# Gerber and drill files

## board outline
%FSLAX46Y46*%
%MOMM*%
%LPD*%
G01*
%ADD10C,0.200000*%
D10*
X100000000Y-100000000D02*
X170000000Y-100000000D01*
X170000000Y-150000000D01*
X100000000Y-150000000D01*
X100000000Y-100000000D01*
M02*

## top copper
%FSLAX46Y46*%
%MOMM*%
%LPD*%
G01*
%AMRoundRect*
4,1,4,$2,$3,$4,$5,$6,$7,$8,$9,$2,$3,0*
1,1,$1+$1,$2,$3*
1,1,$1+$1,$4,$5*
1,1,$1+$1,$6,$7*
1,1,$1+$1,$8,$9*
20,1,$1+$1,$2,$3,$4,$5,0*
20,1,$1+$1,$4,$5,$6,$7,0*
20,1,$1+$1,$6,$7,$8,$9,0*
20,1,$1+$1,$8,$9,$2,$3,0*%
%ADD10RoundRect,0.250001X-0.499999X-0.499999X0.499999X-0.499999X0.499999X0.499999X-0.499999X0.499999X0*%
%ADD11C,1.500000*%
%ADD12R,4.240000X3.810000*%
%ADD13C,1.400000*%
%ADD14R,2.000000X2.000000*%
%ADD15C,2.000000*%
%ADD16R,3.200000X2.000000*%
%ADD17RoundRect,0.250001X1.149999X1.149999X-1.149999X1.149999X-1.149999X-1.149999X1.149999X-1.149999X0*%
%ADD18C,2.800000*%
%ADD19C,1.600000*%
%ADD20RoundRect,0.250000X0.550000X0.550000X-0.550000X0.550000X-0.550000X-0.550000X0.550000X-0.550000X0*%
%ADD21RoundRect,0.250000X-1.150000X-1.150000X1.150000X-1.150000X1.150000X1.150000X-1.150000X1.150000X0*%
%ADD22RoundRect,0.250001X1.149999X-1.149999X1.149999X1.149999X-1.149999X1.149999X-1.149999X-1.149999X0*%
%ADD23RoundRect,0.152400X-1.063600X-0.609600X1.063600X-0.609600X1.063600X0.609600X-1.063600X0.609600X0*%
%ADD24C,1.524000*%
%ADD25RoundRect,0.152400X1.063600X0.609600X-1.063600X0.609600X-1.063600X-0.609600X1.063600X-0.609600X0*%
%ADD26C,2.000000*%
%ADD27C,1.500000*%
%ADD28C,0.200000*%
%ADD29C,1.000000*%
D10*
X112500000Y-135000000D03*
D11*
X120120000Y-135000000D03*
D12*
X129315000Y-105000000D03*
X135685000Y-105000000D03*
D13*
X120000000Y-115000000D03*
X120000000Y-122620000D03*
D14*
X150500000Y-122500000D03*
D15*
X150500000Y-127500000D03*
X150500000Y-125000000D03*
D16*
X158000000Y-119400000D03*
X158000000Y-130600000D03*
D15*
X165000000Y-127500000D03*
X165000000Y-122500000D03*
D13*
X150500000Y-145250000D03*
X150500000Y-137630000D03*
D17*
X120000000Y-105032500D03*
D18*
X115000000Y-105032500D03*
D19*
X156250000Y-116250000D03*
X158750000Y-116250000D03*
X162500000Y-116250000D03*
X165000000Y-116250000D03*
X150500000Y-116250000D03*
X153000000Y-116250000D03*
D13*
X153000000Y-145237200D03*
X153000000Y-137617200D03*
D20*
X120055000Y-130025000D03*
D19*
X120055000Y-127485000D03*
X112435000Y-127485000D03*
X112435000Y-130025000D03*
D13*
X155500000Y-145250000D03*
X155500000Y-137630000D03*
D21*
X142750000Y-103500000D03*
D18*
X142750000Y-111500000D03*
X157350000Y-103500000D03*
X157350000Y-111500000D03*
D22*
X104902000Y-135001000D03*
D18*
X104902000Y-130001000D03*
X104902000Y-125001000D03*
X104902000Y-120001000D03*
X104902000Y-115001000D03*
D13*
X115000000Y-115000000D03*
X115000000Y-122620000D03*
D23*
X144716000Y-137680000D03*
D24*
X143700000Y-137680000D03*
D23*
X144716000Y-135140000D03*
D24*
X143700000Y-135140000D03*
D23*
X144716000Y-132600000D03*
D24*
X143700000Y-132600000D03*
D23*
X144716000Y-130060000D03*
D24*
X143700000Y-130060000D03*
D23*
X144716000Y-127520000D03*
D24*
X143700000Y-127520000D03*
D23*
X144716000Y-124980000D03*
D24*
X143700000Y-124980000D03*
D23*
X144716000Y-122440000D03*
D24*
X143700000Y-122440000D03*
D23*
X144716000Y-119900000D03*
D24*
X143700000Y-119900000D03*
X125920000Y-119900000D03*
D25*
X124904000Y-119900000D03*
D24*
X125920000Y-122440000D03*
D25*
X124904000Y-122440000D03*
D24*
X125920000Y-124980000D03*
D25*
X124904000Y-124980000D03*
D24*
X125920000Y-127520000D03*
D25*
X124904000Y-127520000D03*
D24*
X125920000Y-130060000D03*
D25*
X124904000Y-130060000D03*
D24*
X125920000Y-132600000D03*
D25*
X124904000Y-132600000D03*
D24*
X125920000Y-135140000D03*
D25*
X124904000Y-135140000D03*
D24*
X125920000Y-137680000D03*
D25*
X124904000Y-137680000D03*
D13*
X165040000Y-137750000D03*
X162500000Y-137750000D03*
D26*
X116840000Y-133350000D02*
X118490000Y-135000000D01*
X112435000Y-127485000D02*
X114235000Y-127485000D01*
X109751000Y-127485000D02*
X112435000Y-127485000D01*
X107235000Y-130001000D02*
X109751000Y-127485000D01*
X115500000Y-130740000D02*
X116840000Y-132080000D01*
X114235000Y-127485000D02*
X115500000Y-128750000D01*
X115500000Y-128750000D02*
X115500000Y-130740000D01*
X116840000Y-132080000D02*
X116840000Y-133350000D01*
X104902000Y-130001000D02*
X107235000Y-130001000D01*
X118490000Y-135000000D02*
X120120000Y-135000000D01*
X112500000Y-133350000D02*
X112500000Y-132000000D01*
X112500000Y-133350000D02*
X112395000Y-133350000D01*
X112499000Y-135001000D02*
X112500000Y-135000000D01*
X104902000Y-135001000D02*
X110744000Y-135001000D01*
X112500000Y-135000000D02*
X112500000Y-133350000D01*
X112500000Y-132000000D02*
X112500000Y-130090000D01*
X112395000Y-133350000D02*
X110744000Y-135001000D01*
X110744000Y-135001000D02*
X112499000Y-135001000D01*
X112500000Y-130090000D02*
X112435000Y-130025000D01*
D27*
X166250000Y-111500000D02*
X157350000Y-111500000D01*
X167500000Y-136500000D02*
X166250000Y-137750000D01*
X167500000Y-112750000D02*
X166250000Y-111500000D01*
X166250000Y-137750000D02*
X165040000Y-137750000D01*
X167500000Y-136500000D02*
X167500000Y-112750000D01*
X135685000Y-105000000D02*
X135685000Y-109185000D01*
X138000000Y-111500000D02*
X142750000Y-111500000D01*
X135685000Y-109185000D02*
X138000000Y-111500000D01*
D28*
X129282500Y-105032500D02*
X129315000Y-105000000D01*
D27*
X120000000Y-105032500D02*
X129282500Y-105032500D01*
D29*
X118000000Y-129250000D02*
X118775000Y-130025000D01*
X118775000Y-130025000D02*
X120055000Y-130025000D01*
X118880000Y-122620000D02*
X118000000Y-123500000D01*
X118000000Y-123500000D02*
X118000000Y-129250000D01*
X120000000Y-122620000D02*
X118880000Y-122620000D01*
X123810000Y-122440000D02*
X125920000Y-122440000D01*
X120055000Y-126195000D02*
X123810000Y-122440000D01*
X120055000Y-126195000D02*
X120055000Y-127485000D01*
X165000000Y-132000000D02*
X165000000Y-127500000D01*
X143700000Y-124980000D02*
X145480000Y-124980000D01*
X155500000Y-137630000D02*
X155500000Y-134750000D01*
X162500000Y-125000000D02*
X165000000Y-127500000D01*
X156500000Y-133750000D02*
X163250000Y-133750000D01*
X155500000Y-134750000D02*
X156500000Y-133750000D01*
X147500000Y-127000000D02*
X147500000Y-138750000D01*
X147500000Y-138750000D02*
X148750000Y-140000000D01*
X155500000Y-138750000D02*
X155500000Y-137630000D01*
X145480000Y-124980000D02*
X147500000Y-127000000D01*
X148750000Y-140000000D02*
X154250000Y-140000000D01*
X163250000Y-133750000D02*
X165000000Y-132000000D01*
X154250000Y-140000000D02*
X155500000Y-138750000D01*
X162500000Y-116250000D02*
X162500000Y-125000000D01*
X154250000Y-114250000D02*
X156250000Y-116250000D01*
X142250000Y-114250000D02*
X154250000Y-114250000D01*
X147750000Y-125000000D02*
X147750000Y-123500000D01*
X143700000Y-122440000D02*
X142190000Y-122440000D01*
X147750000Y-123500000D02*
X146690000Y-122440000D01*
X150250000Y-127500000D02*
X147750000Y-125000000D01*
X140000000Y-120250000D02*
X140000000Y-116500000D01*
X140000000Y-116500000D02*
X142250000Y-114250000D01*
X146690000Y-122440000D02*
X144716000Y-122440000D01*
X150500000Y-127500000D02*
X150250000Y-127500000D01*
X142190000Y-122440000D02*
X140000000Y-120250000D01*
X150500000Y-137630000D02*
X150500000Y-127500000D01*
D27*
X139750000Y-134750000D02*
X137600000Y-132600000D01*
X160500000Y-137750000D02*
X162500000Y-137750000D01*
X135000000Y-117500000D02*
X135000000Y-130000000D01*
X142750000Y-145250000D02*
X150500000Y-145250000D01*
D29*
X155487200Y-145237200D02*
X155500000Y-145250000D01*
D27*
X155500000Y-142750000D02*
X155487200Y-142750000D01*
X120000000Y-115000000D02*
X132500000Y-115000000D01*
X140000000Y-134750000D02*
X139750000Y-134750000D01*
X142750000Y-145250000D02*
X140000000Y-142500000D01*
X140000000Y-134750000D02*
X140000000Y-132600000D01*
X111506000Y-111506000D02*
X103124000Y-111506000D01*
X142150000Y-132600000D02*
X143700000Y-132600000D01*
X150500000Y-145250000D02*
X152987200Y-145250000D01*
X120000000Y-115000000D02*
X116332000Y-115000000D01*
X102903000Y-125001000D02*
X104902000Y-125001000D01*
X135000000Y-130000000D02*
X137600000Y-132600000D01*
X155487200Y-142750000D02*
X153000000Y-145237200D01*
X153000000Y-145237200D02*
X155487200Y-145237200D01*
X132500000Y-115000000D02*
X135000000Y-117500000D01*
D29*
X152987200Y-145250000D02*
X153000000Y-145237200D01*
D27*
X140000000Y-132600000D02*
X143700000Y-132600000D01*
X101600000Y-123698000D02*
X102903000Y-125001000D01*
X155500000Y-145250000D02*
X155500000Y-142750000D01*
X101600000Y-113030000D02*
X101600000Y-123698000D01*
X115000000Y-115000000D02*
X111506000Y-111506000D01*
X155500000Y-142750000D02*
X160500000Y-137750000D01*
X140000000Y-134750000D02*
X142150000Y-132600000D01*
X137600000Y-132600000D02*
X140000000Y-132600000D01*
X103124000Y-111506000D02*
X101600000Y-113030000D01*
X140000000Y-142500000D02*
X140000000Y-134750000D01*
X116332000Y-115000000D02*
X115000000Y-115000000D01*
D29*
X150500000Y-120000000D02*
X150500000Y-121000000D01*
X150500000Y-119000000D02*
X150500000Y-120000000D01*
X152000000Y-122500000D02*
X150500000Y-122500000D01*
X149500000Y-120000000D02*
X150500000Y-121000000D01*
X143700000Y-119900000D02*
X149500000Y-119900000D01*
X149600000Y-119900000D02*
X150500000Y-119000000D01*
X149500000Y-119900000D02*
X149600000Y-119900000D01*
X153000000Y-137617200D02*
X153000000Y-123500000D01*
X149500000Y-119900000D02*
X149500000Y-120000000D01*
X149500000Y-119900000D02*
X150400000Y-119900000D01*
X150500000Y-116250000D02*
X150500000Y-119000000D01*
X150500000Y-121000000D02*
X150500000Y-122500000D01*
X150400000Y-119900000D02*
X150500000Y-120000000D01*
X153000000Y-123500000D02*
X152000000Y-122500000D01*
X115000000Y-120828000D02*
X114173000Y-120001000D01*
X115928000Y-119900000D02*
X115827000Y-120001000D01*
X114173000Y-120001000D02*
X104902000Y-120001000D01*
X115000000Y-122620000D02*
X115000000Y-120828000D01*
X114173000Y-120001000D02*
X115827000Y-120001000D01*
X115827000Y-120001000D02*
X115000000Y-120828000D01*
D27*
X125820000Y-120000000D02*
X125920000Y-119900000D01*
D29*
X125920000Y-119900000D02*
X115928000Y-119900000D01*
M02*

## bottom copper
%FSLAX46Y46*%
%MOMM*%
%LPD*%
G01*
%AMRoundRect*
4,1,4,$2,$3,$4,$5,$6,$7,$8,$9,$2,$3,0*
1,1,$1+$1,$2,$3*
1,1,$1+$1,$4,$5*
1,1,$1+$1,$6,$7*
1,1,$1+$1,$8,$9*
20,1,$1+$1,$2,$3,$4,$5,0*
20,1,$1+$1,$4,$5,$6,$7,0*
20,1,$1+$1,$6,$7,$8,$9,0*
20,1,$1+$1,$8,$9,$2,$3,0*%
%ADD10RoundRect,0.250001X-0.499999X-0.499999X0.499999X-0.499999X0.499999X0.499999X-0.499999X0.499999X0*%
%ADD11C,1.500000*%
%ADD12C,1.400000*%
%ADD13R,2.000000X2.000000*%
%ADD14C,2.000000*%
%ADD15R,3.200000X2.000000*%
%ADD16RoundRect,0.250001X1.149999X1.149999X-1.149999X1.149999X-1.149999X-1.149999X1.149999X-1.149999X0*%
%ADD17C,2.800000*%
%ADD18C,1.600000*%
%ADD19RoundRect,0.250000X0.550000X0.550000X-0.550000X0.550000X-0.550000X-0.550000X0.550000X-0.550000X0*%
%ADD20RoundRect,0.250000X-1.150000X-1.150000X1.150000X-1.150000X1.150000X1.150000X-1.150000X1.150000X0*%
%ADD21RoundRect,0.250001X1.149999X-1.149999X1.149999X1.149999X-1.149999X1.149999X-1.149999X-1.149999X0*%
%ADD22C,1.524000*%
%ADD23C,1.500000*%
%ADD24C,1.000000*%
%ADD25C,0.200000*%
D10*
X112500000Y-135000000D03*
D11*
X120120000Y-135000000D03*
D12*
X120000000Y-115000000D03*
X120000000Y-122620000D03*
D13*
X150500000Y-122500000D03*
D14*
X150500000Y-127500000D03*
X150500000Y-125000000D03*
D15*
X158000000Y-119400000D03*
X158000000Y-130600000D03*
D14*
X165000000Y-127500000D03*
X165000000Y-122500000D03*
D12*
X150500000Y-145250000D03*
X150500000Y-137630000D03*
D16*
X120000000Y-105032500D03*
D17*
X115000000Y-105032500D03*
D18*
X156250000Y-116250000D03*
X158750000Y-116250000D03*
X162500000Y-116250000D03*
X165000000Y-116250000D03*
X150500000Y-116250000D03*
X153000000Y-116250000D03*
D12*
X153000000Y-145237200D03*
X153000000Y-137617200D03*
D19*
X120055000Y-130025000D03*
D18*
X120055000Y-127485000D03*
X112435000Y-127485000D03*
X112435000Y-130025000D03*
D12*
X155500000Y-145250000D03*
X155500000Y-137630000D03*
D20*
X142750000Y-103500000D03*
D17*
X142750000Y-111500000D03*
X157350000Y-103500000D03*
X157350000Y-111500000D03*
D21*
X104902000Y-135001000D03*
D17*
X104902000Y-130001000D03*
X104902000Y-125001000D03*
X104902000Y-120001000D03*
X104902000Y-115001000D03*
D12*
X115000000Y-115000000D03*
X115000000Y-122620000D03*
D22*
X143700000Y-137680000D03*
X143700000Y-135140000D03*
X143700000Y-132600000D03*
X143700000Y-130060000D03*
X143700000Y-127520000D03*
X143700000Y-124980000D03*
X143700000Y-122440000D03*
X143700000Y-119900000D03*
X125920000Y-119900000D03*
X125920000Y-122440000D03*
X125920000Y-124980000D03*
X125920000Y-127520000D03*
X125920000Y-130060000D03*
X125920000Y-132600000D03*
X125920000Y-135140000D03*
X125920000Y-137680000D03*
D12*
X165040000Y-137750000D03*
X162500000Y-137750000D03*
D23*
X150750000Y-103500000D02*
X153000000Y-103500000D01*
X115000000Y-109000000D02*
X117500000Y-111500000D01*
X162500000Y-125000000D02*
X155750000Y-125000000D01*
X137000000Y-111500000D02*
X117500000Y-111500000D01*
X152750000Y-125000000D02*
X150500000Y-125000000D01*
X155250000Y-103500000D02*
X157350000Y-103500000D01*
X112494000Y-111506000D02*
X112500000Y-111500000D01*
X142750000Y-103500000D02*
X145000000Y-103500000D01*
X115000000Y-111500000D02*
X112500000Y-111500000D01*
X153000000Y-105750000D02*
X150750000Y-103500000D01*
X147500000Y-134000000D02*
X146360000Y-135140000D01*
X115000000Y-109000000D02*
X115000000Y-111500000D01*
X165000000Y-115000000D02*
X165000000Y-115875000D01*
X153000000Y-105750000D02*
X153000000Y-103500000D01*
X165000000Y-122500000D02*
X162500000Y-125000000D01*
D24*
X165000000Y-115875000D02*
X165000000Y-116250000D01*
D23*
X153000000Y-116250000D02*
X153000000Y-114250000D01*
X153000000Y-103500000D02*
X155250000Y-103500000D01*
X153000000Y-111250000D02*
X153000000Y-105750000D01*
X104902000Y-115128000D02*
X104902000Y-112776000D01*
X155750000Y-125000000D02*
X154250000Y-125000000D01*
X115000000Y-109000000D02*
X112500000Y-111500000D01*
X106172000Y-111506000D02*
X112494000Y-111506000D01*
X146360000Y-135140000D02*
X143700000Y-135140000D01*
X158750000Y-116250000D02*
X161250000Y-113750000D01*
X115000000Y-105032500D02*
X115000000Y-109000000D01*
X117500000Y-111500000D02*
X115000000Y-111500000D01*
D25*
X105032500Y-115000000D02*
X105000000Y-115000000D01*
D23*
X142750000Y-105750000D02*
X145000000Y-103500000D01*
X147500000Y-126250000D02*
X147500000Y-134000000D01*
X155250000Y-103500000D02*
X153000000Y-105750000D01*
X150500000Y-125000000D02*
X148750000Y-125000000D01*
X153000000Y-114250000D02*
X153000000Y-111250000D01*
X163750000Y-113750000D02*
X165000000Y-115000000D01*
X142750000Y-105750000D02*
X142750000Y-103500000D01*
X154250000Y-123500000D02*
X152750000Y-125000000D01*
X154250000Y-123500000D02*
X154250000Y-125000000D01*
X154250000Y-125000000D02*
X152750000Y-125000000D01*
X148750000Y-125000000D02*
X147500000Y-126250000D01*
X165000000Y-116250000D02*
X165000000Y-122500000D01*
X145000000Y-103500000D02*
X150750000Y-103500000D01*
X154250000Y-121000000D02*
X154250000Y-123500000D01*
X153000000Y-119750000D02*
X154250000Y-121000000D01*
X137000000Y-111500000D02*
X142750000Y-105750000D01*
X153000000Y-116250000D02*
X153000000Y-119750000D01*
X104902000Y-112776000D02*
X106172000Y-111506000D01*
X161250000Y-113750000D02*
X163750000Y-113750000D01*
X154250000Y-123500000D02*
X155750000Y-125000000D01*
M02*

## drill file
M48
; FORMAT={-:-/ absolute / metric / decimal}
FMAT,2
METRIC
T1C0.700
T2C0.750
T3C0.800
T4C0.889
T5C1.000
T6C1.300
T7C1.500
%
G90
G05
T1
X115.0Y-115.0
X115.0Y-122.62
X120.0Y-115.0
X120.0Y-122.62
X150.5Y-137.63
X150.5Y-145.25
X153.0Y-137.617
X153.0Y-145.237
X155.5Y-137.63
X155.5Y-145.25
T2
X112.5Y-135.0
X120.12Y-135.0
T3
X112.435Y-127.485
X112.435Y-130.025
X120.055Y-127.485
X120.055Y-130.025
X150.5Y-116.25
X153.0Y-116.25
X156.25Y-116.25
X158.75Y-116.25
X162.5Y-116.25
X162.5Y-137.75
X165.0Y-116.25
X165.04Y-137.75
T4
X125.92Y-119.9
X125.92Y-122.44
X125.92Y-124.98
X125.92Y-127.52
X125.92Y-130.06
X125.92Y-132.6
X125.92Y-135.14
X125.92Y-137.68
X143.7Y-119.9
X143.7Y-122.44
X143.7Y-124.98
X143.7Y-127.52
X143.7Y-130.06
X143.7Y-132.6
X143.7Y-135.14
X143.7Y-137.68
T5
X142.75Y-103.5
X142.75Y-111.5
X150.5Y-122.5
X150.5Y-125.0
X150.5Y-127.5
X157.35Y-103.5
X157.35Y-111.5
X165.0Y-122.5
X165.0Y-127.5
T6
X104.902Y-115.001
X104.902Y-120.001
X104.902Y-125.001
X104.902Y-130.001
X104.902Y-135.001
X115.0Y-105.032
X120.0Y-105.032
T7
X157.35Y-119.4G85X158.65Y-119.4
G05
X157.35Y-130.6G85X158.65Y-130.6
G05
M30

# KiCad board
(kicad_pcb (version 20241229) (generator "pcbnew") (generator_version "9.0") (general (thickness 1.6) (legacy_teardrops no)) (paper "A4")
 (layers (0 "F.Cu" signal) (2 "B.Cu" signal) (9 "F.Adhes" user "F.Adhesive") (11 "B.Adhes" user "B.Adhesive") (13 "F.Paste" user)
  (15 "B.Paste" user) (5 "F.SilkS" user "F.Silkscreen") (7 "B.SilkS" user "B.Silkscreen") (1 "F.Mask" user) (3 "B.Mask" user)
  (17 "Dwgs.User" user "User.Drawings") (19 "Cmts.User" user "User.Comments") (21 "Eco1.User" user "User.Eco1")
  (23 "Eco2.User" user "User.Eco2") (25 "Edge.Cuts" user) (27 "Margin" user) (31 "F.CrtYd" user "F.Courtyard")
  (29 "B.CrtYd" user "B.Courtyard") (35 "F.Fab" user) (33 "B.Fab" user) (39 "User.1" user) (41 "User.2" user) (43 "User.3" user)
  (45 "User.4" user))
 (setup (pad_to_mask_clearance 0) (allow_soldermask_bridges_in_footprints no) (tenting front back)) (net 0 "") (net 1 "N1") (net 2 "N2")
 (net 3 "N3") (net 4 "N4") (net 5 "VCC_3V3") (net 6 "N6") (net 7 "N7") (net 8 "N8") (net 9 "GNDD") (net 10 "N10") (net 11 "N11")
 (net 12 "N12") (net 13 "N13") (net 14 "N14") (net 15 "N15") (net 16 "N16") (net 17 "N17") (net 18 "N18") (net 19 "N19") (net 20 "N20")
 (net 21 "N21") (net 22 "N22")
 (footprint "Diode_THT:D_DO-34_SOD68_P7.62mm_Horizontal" (layer "F.Cu") (at 112.5 135)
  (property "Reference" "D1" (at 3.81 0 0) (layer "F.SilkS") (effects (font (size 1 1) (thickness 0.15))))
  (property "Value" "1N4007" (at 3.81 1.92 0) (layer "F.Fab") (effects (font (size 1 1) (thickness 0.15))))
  (pad "1" thru_hole roundrect (at 0 0) (size 1.5 1.5) (drill 0.75) (layers "*.Cu" "*.Mask") (remove_unused_layers no)
   (roundrect_rratio 0.166667) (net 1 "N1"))
  (pad "2" thru_hole circle (at 7.62 0) (size 1.5 1.5) (drill 0.75) (layers "*.Cu" "*.Mask") (remove_unused_layers no) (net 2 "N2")))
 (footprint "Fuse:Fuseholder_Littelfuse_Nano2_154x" (layer "F.Cu") (at 132.5 105)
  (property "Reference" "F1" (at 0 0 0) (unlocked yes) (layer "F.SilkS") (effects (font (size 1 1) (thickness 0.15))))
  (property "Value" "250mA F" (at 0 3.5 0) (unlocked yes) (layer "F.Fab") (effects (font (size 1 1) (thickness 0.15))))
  (pad "1" smd rect (at -3.185 0) (size 4.24 3.81) (layers "F.Cu" "F.Mask" "F.Paste") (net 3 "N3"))
  (pad "2" smd rect (at 3.185 0) (size 4.24 3.81) (layers "F.Cu" "F.Mask" "F.Paste") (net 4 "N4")))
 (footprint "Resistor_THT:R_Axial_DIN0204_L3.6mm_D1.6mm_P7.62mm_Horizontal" (layer "F.Cu") (at 120 115 -90)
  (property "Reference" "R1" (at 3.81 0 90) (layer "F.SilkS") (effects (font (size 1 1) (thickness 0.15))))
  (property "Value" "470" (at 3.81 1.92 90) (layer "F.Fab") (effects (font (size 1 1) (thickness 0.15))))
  (pad "1" thru_hole circle (at 0 0 270) (size 1.4 1.4) (drill 0.7) (layers "*.Cu" "*.Mask") (remove_unused_layers no) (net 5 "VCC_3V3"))
  (pad "2" thru_hole circle (at 7.62 0 270) (size 1.4 1.4) (drill 0.7) (layers "*.Cu" "*.Mask") (remove_unused_layers no) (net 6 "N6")))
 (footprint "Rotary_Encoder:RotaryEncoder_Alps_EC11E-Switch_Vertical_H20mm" (layer "F.Cu") (at 150.5 122.5)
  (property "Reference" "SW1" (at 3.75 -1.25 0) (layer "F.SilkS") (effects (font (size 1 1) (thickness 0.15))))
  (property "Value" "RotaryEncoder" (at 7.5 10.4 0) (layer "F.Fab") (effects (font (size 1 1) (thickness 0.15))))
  (pad "A" thru_hole rect (at 0 0) (size 2 2) (drill 1) (layers "*.Cu" "*.Mask") (remove_unused_layers no) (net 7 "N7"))
  (pad "B" thru_hole circle (at 0 5) (size 2 2) (drill 1) (layers "*.Cu" "*.Mask") (remove_unused_layers no) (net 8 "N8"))
  (pad "C" thru_hole circle (at 0 2.5) (size 2 2) (drill 1) (layers "*.Cu" "*.Mask") (remove_unused_layers no) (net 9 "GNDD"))
  (pad "MP" thru_hole rect (at 7.5 -3.1) (size 3.2 2) (drill oval 2.8 1.5) (layers "*.Cu" "*.Mask") (remove_unused_layers no))
  (pad "MP" thru_hole rect (at 7.5 8.1) (size 3.2 2) (drill oval 2.8 1.5) (layers "*.Cu" "*.Mask") (remove_unused_layers no))
  (pad "S1" thru_hole circle (at 14.5 5) (size 2 2) (drill 1) (layers "*.Cu" "*.Mask") (remove_unused_layers no) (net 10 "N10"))
  (pad "S2" thru_hole circle (at 14.5 0) (size 2 2) (drill 1) (layers "*.Cu" "*.Mask") (remove_unused_layers no) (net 9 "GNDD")))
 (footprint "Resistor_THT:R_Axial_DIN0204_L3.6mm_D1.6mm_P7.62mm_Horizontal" (layer "F.Cu") (at 150.5 145.25 90)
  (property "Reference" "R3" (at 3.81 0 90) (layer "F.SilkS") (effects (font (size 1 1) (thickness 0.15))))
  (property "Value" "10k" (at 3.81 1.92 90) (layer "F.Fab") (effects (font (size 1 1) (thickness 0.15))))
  (pad "1" thru_hole circle (at 0 0 90) (size 1.4 1.4) (drill 0.7) (layers "*.Cu" "*.Mask") (remove_unused_layers no) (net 5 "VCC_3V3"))
  (pad "2" thru_hole circle (at 7.62 0 90) (size 1.4 1.4) (drill 0.7) (layers "*.Cu" "*.Mask") (remove_unused_layers no) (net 8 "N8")))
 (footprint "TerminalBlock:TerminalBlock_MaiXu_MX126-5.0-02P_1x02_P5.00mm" (layer "F.Cu") (at 120 105.0325 180)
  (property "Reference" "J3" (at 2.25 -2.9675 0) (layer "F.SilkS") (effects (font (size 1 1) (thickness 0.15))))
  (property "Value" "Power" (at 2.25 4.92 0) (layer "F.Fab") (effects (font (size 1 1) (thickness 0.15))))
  (pad "1" thru_hole roundrect (at 0 0 180) (size 2.8 2.8) (drill 1.3) (layers "*.Cu" "*.Mask") (remove_unused_layers no)
   (roundrect_rratio 0.089286) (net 3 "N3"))
  (pad "2" thru_hole circle (at 5 0 180) (size 2.8 2.8) (drill 1.3) (layers "*.Cu" "*.Mask") (remove_unused_layers no) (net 9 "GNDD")))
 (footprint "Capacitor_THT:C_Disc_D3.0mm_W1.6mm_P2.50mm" (layer "F.Cu") (at 156.25 116.25)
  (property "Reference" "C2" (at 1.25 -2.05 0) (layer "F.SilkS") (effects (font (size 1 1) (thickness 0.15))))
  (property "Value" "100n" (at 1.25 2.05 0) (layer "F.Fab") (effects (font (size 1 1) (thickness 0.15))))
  (pad "1" thru_hole circle (at 0 0) (size 1.6 1.6) (drill 0.8) (layers "*.Cu" "*.Mask") (remove_unused_layers no) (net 8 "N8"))
  (pad "2" thru_hole circle (at 2.5 0) (size 1.6 1.6) (drill 0.8) (layers "*.Cu" "*.Mask") (remove_unused_layers no) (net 9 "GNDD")))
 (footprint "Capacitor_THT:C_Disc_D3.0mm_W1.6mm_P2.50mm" (layer "F.Cu") (at 162.5 116.25)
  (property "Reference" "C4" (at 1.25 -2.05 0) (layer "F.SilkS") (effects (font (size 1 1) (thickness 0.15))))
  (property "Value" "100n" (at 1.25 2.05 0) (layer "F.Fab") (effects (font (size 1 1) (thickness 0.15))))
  (pad "1" thru_hole circle (at 0 0) (size 1.6 1.6) (drill 0.8) (layers "*.Cu" "*.Mask") (remove_unused_layers no) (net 10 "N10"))
  (pad "2" thru_hole circle (at 2.5 0) (size 1.6 1.6) (drill 0.8) (layers "*.Cu" "*.Mask") (remove_unused_layers no) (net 9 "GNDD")))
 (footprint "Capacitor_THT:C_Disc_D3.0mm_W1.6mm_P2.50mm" (layer "F.Cu") (at 150.5 116.25)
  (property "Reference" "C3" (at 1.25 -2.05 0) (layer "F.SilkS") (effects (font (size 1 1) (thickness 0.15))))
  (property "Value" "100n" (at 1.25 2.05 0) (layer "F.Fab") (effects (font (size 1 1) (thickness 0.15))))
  (pad "1" thru_hole circle (at 0 0) (size 1.6 1.6) (drill 0.8) (layers "*.Cu" "*.Mask") (remove_unused_layers no) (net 7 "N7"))
  (pad "2" thru_hole circle (at 2.5 0) (size 1.6 1.6) (drill 0.8) (layers "*.Cu" "*.Mask") (remove_unused_layers no) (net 9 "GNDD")))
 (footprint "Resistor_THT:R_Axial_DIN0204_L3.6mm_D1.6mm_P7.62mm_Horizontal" (layer "F.Cu") (at 153 145.2372 90)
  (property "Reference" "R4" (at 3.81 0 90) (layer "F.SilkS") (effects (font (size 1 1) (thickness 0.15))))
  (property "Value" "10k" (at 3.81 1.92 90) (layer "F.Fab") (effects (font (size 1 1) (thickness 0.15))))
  (pad "1" thru_hole circle (at 0 0 90) (size 1.4 1.4) (drill 0.7) (layers "*.Cu" "*.Mask") (remove_unused_layers no) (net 5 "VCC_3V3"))
  (pad "2" thru_hole circle (at 7.62 0 90) (size 1.4 1.4) (drill 0.7) (layers "*.Cu" "*.Mask") (remove_unused_layers no) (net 7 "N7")))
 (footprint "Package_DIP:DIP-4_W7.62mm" (layer "F.Cu") (at 120.055 130.025 180)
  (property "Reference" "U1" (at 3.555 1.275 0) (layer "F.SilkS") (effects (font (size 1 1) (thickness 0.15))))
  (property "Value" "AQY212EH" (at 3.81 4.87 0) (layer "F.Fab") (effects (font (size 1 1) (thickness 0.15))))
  (pad "1" thru_hole roundrect (at 0 0 180) (size 1.6 1.6) (drill 0.8) (layers "*.Cu" "*.Mask") (remove_unused_layers no)
   (roundrect_rratio 0.15625) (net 6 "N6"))
  (pad "2" thru_hole circle (at 0 2.54 180) (size 1.6 1.6) (drill 0.8) (layers "*.Cu" "*.Mask") (remove_unused_layers no) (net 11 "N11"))
  (pad "3" thru_hole circle (at 7.62 2.54 180) (size 1.6 1.6) (drill 0.8) (layers "*.Cu" "*.Mask") (remove_unused_layers no) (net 2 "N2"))
  (pad "4" thru_hole circle (at 7.62 0 180) (size 1.6 1.6) (drill 0.8) (layers "*.Cu" "*.Mask") (remove_unused_layers no) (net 1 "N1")))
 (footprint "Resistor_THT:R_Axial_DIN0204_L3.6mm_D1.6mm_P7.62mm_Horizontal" (layer "F.Cu") (at 155.5 145.25 90)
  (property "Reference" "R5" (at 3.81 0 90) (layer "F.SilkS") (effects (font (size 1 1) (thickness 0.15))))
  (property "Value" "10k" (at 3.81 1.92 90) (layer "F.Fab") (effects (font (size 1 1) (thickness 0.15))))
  (pad "1" thru_hole circle (at 0 0 90) (size 1.4 1.4) (drill 0.7) (layers "*.Cu" "*.Mask") (remove_unused_layers no) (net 5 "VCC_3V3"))
  (pad "2" thru_hole circle (at 7.62 0 90) (size 1.4 1.4) (drill 0.7) (layers "*.Cu" "*.Mask") (remove_unused_layers no) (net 10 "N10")))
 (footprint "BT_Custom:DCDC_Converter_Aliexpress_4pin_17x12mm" (layer "F.Cu") (at 150.05 107.5)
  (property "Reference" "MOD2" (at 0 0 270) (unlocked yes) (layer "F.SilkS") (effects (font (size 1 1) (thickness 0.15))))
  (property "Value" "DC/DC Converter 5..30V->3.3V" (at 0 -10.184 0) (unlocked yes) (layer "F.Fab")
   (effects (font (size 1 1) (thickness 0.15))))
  (pad "1" thru_hole roundrect (at -7.3 -4) (size 2.8 2.8) (drill 1) (layers "*.Cu" "*.Mask") (remove_unused_layers no)
   (roundrect_rratio 0.08928571429) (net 9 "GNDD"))
  (pad "2" thru_hole circle (at -7.3 4) (size 2.8 2.8) (drill 1) (layers "*.Cu" "*.Mask") (remove_unused_layers no) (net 4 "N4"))
  (pad "3" thru_hole circle (at 7.3 -4) (size 2.8 2.8) (drill 1) (layers "*.Cu" "*.Mask") (remove_unused_layers no) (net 9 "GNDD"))
  (pad "4" thru_hole circle (at 7.3 4) (size 2.8 2.8) (drill 1) (layers "*.Cu" "*.Mask") (remove_unused_layers no) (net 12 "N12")))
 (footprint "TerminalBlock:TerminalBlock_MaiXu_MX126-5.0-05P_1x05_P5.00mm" (layer "F.Cu") (at 104.902 135.001 90)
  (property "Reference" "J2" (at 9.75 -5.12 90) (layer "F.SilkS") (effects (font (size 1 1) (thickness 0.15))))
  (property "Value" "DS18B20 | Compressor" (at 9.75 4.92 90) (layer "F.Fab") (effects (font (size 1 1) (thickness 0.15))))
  (pad "1" thru_hole roundrect (at 0 0 90) (size 2.8 2.8) (drill 1.3) (layers "*.Cu" "*.Mask") (remove_unused_layers no)
   (roundrect_rratio 0.089286) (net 1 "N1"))
  (pad "2" thru_hole circle (at 5 0 90) (size 2.8 2.8) (drill 1.3) (layers "*.Cu" "*.Mask") (remove_unused_layers no) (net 2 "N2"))
  (pad "3" thru_hole circle (at 10 0 90) (size 2.8 2.8) (drill 1.3) (layers "*.Cu" "*.Mask") (remove_unused_layers no) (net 5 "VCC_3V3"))
  (pad "4" thru_hole circle (at 15 0 90) (size 2.8 2.8) (drill 1.3) (layers "*.Cu" "*.Mask") (remove_unused_layers no) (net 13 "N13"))
  (pad "5" thru_hole circle (at 20 0 90) (size 2.8 2.8) (drill 1.3) (layers "*.Cu" "*.Mask") (remove_unused_layers no) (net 9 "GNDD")))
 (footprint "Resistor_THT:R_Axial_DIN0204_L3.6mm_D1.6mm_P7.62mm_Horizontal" (layer "F.Cu") (at 115 115 -90)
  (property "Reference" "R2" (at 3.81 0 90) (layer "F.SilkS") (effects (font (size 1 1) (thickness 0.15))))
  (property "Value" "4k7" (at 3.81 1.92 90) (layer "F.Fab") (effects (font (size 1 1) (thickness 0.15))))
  (pad "1" thru_hole circle (at 0 0 270) (size 1.4 1.4) (drill 0.7) (layers "*.Cu" "*.Mask") (remove_unused_layers no) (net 5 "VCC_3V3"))
  (pad "2" thru_hole circle (at 7.62 0 270) (size 1.4 1.4) (drill 0.7) (layers "*.Cu" "*.Mask") (remove_unused_layers no) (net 13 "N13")))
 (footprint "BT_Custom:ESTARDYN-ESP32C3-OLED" (layer "F.Cu") (at 134.81 130.06 180)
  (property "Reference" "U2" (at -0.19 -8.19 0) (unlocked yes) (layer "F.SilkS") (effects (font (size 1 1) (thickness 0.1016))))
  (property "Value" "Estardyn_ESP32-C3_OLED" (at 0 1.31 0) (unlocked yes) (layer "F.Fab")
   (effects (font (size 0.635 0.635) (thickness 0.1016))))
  (pad "1" smd roundrect (at -9.906 -7.62) (size 2.432 1.524) (layers "F.Cu" "F.Mask") (roundrect_rratio 0.1) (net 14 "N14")
   (thermal_bridge_angle 45))
  (pad "1" thru_hole circle (at -8.89 -7.62) (size 1.524 1.524) (drill 0.889) (layers "*.Cu" "*.Mask") (remove_unused_layers no)
   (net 14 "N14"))
  (pad "2" smd roundrect (at -9.906 -5.08) (size 2.432 1.524) (layers "F.Cu" "F.Mask") (roundrect_rratio 0.1) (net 9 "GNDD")
   (thermal_bridge_angle 45))
  (pad "2" thru_hole circle (at -8.89 -5.08) (size 1.524 1.524) (drill 0.889) (layers "*.Cu" "*.Mask") (remove_unused_layers no)
   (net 9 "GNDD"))
  (pad "3" smd roundrect (at -9.906 -2.54) (size 2.432 1.524) (layers "F.Cu" "F.Mask") (roundrect_rratio 0.1) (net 5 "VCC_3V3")
   (thermal_bridge_angle 45))
  (pad "3" thru_hole circle (at -8.89 -2.54) (size 1.524 1.524) (drill 0.889) (layers "*.Cu" "*.Mask") (remove_unused_layers no)
   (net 5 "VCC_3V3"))
  (pad "4" smd roundrect (at -9.906 0) (size 2.432 1.524) (layers "F.Cu" "F.Mask") (roundrect_rratio 0.1) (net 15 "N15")
   (thermal_bridge_angle 45))
  (pad "4" thru_hole circle (at -8.89 0) (size 1.524 1.524) (drill 0.889) (layers "*.Cu" "*.Mask") (remove_unused_layers no) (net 15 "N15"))
  (pad "5" smd roundrect (at -9.906 2.54) (size 2.432 1.524) (layers "F.Cu" "F.Mask") (roundrect_rratio 0.1) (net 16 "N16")
   (thermal_bridge_angle 45))
  (pad "5" thru_hole circle (at -8.89 2.54) (size 1.524 1.524) (drill 0.889) (layers "*.Cu" "*.Mask") (remove_unused_layers no)
   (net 16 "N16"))
  (pad "6" smd roundrect (at -9.906 5.08) (size 2.432 1.524) (layers "F.Cu" "F.Mask") (roundrect_rratio 0.1) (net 10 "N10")
   (thermal_bridge_angle 45))
  (pad "6" thru_hole circle (at -8.89 5.08) (size 1.524 1.524) (drill 0.889) (layers "*.Cu" "*.Mask") (remove_unused_layers no)
   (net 10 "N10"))
  (pad "7" smd roundrect (at -9.906 7.62) (size 2.432 1.524) (layers "F.Cu" "F.Mask") (roundrect_rratio 0.1) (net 8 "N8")
   (thermal_bridge_angle 45))
  (pad "7" thru_hole circle (at -8.89 7.62) (size 1.524 1.524) (drill 0.889) (layers "*.Cu" "*.Mask") (remove_unused_layers no) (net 8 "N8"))
  (pad "8" smd roundrect (at -9.906 10.16) (size 2.432 1.524) (layers "F.Cu" "F.Mask") (roundrect_rratio 0.1) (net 7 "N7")
   (thermal_bridge_angle 45))
  (pad "8" thru_hole circle (at -8.89 10.16 180) (size 1.524 1.524) (drill 0.889) (layers "*.Cu" "*.Mask") (remove_unused_layers no)
   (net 7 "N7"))
  (pad "9" thru_hole circle (at 8.89 10.16 180) (size 1.524 1.524) (drill 0.889) (layers "*.Cu" "*.Mask") (remove_unused_layers no)
   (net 13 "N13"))
  (pad "9" smd roundrect (at 9.906 10.16 180) (size 2.432 1.524) (layers "F.Cu" "F.Mask") (roundrect_rratio 0.1) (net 13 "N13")
   (thermal_bridge_angle 45))
  (pad "10" thru_hole circle (at 8.89 7.62 180) (size 1.524 1.524) (drill 0.889) (layers "*.Cu" "*.Mask") (remove_unused_layers no)
   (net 11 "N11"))
  (pad "10" smd roundrect (at 9.906 7.62 180) (size 2.432 1.524) (layers "F.Cu" "F.Mask") (roundrect_rratio 0.1) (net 11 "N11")
   (thermal_bridge_angle 45))
  (pad "11" thru_hole circle (at 8.89 5.08 180) (size 1.524 1.524) (drill 0.889) (layers "*.Cu" "*.Mask") (remove_unused_layers no)
   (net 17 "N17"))
  (pad "11" smd roundrect (at 9.906 5.08 180) (size 2.432 1.524) (layers "F.Cu" "F.Mask") (roundrect_rratio 0.1) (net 17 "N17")
   (thermal_bridge_angle 45))
  (pad "12" thru_hole circle (at 8.89 2.54 180) (size 1.524 1.524) (drill 0.889) (layers "*.Cu" "*.Mask") (remove_unused_layers no)
   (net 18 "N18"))
  (pad "12" smd roundrect (at 9.906 2.54 180) (size 2.432 1.524) (layers "F.Cu" "F.Mask") (roundrect_rratio 0.1) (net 18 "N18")
   (thermal_bridge_angle 45))
  (pad "13" thru_hole circle (at 8.89 0 180) (size 1.524 1.524) (drill 0.889) (layers "*.Cu" "*.Mask") (remove_unused_layers no)
   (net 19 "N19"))
  (pad "13" smd roundrect (at 9.906 0 180) (size 2.432 1.524) (layers "F.Cu" "F.Mask") (roundrect_rratio 0.1) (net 19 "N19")
   (thermal_bridge_angle 45))
  (pad "14" thru_hole circle (at 8.89 -2.54 180) (size 1.524 1.524) (drill 0.889) (layers "*.Cu" "*.Mask") (remove_unused_layers no)
   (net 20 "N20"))
  (pad "14" smd roundrect (at 9.906 -2.54 180) (size 2.432 1.524) (layers "F.Cu" "F.Mask") (roundrect_rratio 0.1) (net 20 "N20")
   (thermal_bridge_angle 45))
  (pad "15" thru_hole circle (at 8.89 -5.08 180) (size 1.524 1.524) (drill 0.889) (layers "*.Cu" "*.Mask") (remove_unused_layers no)
   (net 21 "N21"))
  (pad "15" smd roundrect (at 9.906 -5.08 180) (size 2.432 1.524) (layers "F.Cu" "F.Mask") (roundrect_rratio 0.1) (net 21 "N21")
   (thermal_bridge_angle 45))
  (pad "16" thru_hole circle (at 8.89 -7.62 180) (size 1.524 1.524) (drill 0.889) (layers "*.Cu" "*.Mask") (remove_unused_layers no)
   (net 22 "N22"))
  (pad "16" smd roundrect (at 9.906 -7.62 180) (size 2.432 1.524) (layers "F.Cu" "F.Mask") (roundrect_rratio 0.1) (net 22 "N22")
   (thermal_bridge_angle 45)))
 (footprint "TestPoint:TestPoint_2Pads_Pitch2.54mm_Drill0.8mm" (layer "F.Cu") (at 165.04 137.75 180)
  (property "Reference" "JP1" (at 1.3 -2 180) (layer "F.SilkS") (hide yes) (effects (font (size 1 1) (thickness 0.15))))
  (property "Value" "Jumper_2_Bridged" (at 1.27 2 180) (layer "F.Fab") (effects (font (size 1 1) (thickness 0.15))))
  (pad "1" thru_hole circle (at 0 0 180) (size 1.4 1.4) (drill 0.8) (layers "*.Cu" "*.Mask") (remove_unused_layers no) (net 12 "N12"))
  (pad "2" thru_hole circle (at 2.54 0 180) (size 1.4 1.4) (drill 0.8) (layers "*.Cu" "*.Mask") (remove_unused_layers no) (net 5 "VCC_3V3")))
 (gr_rect (start 100 100) (end 170 150) (stroke (width 0.2) (type solid)) (fill no) (layer "Edge.Cuts"))
 (segment (start 116.84 133.35) (end 118.49 135) (width 2) (layer "F.Cu") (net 2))
 (segment (start 112.435 127.485) (end 114.235 127.485) (width 2) (layer "F.Cu") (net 2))
 (segment (start 109.751 127.485) (end 112.435 127.485) (width 2) (layer "F.Cu") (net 2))
 (segment (start 107.235 130.001) (end 109.751 127.485) (width 2) (layer "F.Cu") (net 2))
 (segment (start 115.5 130.74) (end 116.84 132.08) (width 2) (layer "F.Cu") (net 2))
 (segment (start 114.235 127.485) (end 115.5 128.75) (width 2) (layer "F.Cu") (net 2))
 (segment (start 115.5 128.75) (end 115.5 130.74) (width 2) (layer "F.Cu") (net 2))
 (segment (start 116.84 132.08) (end 116.84 133.35) (width 2) (layer "F.Cu") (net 2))
 (segment (start 104.902 130.001) (end 107.235 130.001) (width 2) (layer "F.Cu") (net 2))
 (segment (start 118.49 135) (end 120.12 135) (width 2) (layer "F.Cu") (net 2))
 (segment (start 112.5 133.35) (end 112.5 132) (width 2) (layer "F.Cu") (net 1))
 (segment (start 112.5 133.35) (end 112.395 133.35) (width 2) (layer "F.Cu") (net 1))
 (segment (start 112.499 135.001) (end 112.5 135) (width 2) (layer "F.Cu") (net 1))
 (segment (start 104.902 135.001) (end 110.744 135.001) (width 2) (layer "F.Cu") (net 1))
 (segment (start 112.5 135) (end 112.5 133.35) (width 2) (layer "F.Cu") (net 1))
 (segment (start 112.5 132) (end 112.5 130.09) (width 2) (layer "F.Cu") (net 1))
 (segment (start 112.395 133.35) (end 110.744 135.001) (width 2) (layer "F.Cu") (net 1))
 (segment (start 110.744 135.001) (end 112.499 135.001) (width 2) (layer "F.Cu") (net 1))
 (segment (start 112.5 130.09) (end 112.435 130.025) (width 2) (layer "F.Cu") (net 1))
 (segment (start 166.25 111.5) (end 157.35 111.5) (width 1.5) (layer "F.Cu") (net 12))
 (segment (start 167.5 136.5) (end 166.25 137.75) (width 1.5) (layer "F.Cu") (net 12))
 (segment (start 167.5 112.75) (end 166.25 111.5) (width 1.5) (layer "F.Cu") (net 12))
 (segment (start 166.25 137.75) (end 165.04 137.75) (width 1.5) (layer "F.Cu") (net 12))
 (segment (start 167.5 136.5) (end 167.5 112.75) (width 1.5) (layer "F.Cu") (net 12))
 (segment (start 135.685 105) (end 135.685 109.185) (width 1.5) (layer "F.Cu") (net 4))
 (segment (start 138 111.5) (end 142.75 111.5) (width 1.5) (layer "F.Cu") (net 4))
 (segment (start 135.685 109.185) (end 138 111.5) (width 1.5) (layer "F.Cu") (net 4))
 (segment (start 129.2825 105.0325) (end 129.315 105) (width 0.2) (layer "F.Cu") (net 3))
 (segment (start 120 105.0325) (end 129.2825 105.0325) (width 1.5) (layer "F.Cu") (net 3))
 (segment (start 150.75 103.5) (end 153 103.5) (width 1.5) (layer "B.Cu") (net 9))
 (segment (start 115 109) (end 117.5 111.5) (width 1.5) (layer "B.Cu") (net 9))
 (segment (start 162.5 125) (end 155.75 125) (width 1.5) (layer "B.Cu") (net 9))
 (segment (start 137 111.5) (end 117.5 111.5) (width 1.5) (layer "B.Cu") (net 9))
 (segment (start 152.75 125) (end 150.5 125) (width 1.5) (layer "B.Cu") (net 9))
 (segment (start 155.25 103.5) (end 157.35 103.5) (width 1.5) (layer "B.Cu") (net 9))
 (segment (start 112.494 111.506) (end 112.5 111.5) (width 1.5) (layer "B.Cu") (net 9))
 (segment (start 142.75 103.5) (end 145 103.5) (width 1.5) (layer "B.Cu") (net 9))
 (segment (start 115 111.5) (end 112.5 111.5) (width 1.5) (layer "B.Cu") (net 9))
 (segment (start 153 105.75) (end 150.75 103.5) (width 1.5) (layer "B.Cu") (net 9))
 (segment (start 147.5 134) (end 146.36 135.14) (width 1.5) (layer "B.Cu") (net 9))
 (segment (start 115 109) (end 115 111.5) (width 1.5) (layer "B.Cu") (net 9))
 (segment (start 165 115) (end 165 115.875) (width 1.5) (layer "B.Cu") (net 9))
 (segment (start 153 105.75) (end 153 103.5) (width 1.5) (layer "B.Cu") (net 9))
 (segment (start 165 122.5) (end 162.5 125) (width 1.5) (layer "B.Cu") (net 9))
 (segment (start 165 115.875) (end 165 116.25) (width 1) (layer "B.Cu") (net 9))
 (segment (start 153 116.25) (end 153 114.25) (width 1.5) (layer "B.Cu") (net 9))
 (segment (start 153 103.5) (end 155.25 103.5) (width 1.5) (layer "B.Cu") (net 9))
 (segment (start 153 111.25) (end 153 105.75) (width 1.5) (layer "B.Cu") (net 9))
 (segment (start 104.902 115.128) (end 104.902 112.776) (width 1.5) (layer "B.Cu") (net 9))
 (segment (start 155.75 125) (end 154.25 125) (width 1.5) (layer "B.Cu") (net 9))
 (segment (start 115 109) (end 112.5 111.5) (width 1.5) (layer "B.Cu") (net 9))
 (segment (start 106.172 111.506) (end 112.494 111.506) (width 1.5) (layer "B.Cu") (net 9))
 (segment (start 146.36 135.14) (end 143.7 135.14) (width 1.5) (layer "B.Cu") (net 9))
 (segment (start 158.75 116.25) (end 161.25 113.75) (width 1.5) (layer "B.Cu") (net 9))
 (segment (start 115 105.0325) (end 115 109) (width 1.5) (layer "B.Cu") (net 9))
 (segment (start 117.5 111.5) (end 115 111.5) (width 1.5) (layer "B.Cu") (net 9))
 (segment (start 105.0325 115) (end 105 115) (width 0.2) (layer "B.Cu") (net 9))
 (segment (start 142.75 105.75) (end 145 103.5) (width 1.5) (layer "B.Cu") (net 9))
 (segment (start 147.5 126.25) (end 147.5 134) (width 1.5) (layer "B.Cu") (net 9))
 (segment (start 155.25 103.5) (end 153 105.75) (width 1.5) (layer "B.Cu") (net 9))
 (segment (start 150.5 125) (end 148.75 125) (width 1.5) (layer "B.Cu") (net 9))
 (segment (start 153 114.25) (end 153 111.25) (width 1.5) (layer "B.Cu") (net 9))
 (segment (start 163.75 113.75) (end 165 115) (width 1.5) (layer "B.Cu") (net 9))
 (segment (start 142.75 105.75) (end 142.75 103.5) (width 1.5) (layer "B.Cu") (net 9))
 (segment (start 154.25 123.5) (end 152.75 125) (width 1.5) (layer "B.Cu") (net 9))
 (segment (start 154.25 123.5) (end 154.25 125) (width 1.5) (layer "B.Cu") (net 9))
 (segment (start 154.25 125) (end 152.75 125) (width 1.5) (layer "B.Cu") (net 9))
 (segment (start 148.75 125) (end 147.5 126.25) (width 1.5) (layer "B.Cu") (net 9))
 (segment (start 165 116.25) (end 165 122.5) (width 1.5) (layer "B.Cu") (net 9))
 (segment (start 145 103.5) (end 150.75 103.5) (width 1.5) (layer "B.Cu") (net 9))
 (segment (start 154.25 121) (end 154.25 123.5) (width 1.5) (layer "B.Cu") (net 9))
 (segment (start 153 119.75) (end 154.25 121) (width 1.5) (layer "B.Cu") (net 9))
 (segment (start 137 111.5) (end 142.75 105.75) (width 1.5) (layer "B.Cu") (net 9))
 (segment (start 153 116.25) (end 153 119.75) (width 1.5) (layer "B.Cu") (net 9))
 (segment (start 104.902 112.776) (end 106.172 111.506) (width 1.5) (layer "B.Cu") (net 9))
 (segment (start 161.25 113.75) (end 163.75 113.75) (width 1.5) (layer "B.Cu") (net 9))
 (segment (start 154.25 123.5) (end 155.75 125) (width 1.5) (layer "B.Cu") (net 9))
 (segment (start 118 129.25) (end 118.775 130.025) (width 1) (layer "F.Cu") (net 6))
 (segment (start 118.775 130.025) (end 120.055 130.025) (width 1) (layer "F.Cu") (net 6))
 (segment (start 118.88 122.62) (end 118 123.5) (width 1) (layer "F.Cu") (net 6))
 (segment (start 118 123.5) (end 118 129.25) (width 1) (layer "F.Cu") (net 6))
 (segment (start 120 122.62) (end 118.88 122.62) (width 1) (layer "F.Cu") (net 6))
 (segment (start 123.81 122.44) (end 125.92 122.44) (width 1) (layer "F.Cu") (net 11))
 (segment (start 120.055 126.195) (end 123.81 122.44) (width 1) (layer "F.Cu") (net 11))
 (segment (start 120.055 126.195) (end 120.055 127.485) (width 1) (layer "F.Cu") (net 11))
 (segment (start 165 132) (end 165 127.5) (width 1) (layer "F.Cu") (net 10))
 (segment (start 143.7 124.98) (end 145.48 124.98) (width 1) (layer "F.Cu") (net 10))
 (segment (start 155.5 137.63) (end 155.5 134.75) (width 1) (layer "F.Cu") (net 10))
 (segment (start 162.5 125) (end 165 127.5) (width 1) (layer "F.Cu") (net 10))
 (segment (start 156.5 133.75) (end 163.25 133.75) (width 1) (layer "F.Cu") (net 10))
 (segment (start 155.5 134.75) (end 156.5 133.75) (width 1) (layer "F.Cu") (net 10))
 (segment (start 147.5 127) (end 147.5 138.75) (width 1) (layer "F.Cu") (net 10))
 (segment (start 147.5 138.75) (end 148.75 140) (width 1) (layer "F.Cu") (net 10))
 (segment (start 155.5 138.75) (end 155.5 137.63) (width 1) (layer "F.Cu") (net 10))
 (segment (start 145.48 124.98) (end 147.5 127) (width 1) (layer "F.Cu") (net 10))
 (segment (start 148.75 140) (end 154.25 140) (width 1) (layer "F.Cu") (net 10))
 (segment (start 163.25 133.75) (end 165 132) (width 1) (layer "F.Cu") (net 10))
 (segment (start 154.25 140) (end 155.5 138.75) (width 1) (layer "F.Cu") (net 10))
 (segment (start 162.5 116.25) (end 162.5 125) (width 1) (layer "F.Cu") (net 10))
 (segment (start 154.25 114.25) (end 156.25 116.25) (width 1) (layer "F.Cu") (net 8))
 (segment (start 142.25 114.25) (end 154.25 114.25) (width 1) (layer "F.Cu") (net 8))
 (segment (start 147.75 125) (end 147.75 123.5) (width 1) (layer "F.Cu") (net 8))
 (segment (start 143.7 122.44) (end 142.19 122.44) (width 1) (layer "F.Cu") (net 8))
 (segment (start 147.75 123.5) (end 146.69 122.44) (width 1) (layer "F.Cu") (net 8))
 (segment (start 150.25 127.5) (end 147.75 125) (width 1) (layer "F.Cu") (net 8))
 (segment (start 140 120.25) (end 140 116.5) (width 1) (layer "F.Cu") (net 8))
 (segment (start 140 116.5) (end 142.25 114.25) (width 1) (layer "F.Cu") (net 8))
 (segment (start 146.69 122.44) (end 144.716 122.44) (width 1) (layer "F.Cu") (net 8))
 (segment (start 150.5 127.5) (end 150.25 127.5) (width 1) (layer "F.Cu") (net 8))
 (segment (start 142.19 122.44) (end 140 120.25) (width 1) (layer "F.Cu") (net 8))
 (segment (start 150.5 137.63) (end 150.5 127.5) (width 1) (layer "F.Cu") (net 8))
 (segment (start 139.75 134.75) (end 137.6 132.6) (width 1.5) (layer "F.Cu") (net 5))
 (segment (start 160.5 137.75) (end 162.5 137.75) (width 1.5) (layer "F.Cu") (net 5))
 (segment (start 135 117.5) (end 135 130) (width 1.5) (layer "F.Cu") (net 5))
 (segment (start 142.75 145.25) (end 150.5 145.25) (width 1.5) (layer "F.Cu") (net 5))
 (segment (start 155.4872 145.2372) (end 155.5 145.25) (width 1) (layer "F.Cu") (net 5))
 (segment (start 155.5 142.75) (end 155.4872 142.75) (width 1.5) (layer "F.Cu") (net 5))
 (segment (start 120 115) (end 132.5 115) (width 1.5) (layer "F.Cu") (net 5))
 (segment (start 140 134.75) (end 139.75 134.75) (width 1.5) (layer "F.Cu") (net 5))
 (segment (start 142.75 145.25) (end 140 142.5) (width 1.5) (layer "F.Cu") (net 5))
 (segment (start 140 134.75) (end 140 132.6) (width 1.5) (layer "F.Cu") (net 5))
 (segment (start 111.506 111.506) (end 103.124 111.506) (width 1.5) (layer "F.Cu") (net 5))
 (segment (start 142.15 132.6) (end 143.7 132.6) (width 1.5) (layer "F.Cu") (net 5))
 (segment (start 150.5 145.25) (end 152.9872 145.25) (width 1.5) (layer "F.Cu") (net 5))
 (segment (start 120 115) (end 116.332 115) (width 1.5) (layer "F.Cu") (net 5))
 (segment (start 102.903 125.001) (end 104.902 125.001) (width 1.5) (layer "F.Cu") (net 5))
 (segment (start 135 130) (end 137.6 132.6) (width 1.5) (layer "F.Cu") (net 5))
 (segment (start 155.4872 142.75) (end 153 145.2372) (width 1.5) (layer "F.Cu") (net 5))
 (segment (start 153 145.2372) (end 155.4872 145.2372) (width 1.5) (layer "F.Cu") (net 5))
 (segment (start 132.5 115) (end 135 117.5) (width 1.5) (layer "F.Cu") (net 5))
 (segment (start 152.9872 145.25) (end 153 145.2372) (width 1) (layer "F.Cu") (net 5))
 (segment (start 140 132.6) (end 143.7 132.6) (width 1.5) (layer "F.Cu") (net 5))
 (segment (start 101.6 123.698) (end 102.903 125.001) (width 1.5) (layer "F.Cu") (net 5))
 (segment (start 155.5 145.25) (end 155.5 142.75) (width 1.5) (layer "F.Cu") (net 5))
 (segment (start 101.6 113.03) (end 101.6 123.698) (width 1.5) (layer "F.Cu") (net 5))
 (segment (start 115 115) (end 111.506 111.506) (width 1.5) (layer "F.Cu") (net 5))
 (segment (start 155.5 142.75) (end 160.5 137.75) (width 1.5) (layer "F.Cu") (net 5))
 (segment (start 140 134.75) (end 142.15 132.6) (width 1.5) (layer "F.Cu") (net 5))
 (segment (start 137.6 132.6) (end 140 132.6) (width 1.5) (layer "F.Cu") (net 5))
 (segment (start 103.124 111.506) (end 101.6 113.03) (width 1.5) (layer "F.Cu") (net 5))
 (segment (start 140 142.5) (end 140 134.75) (width 1.5) (layer "F.Cu") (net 5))
 (segment (start 116.332 115) (end 115 115) (width 1.5) (layer "F.Cu") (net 5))
 (segment (start 150.5 120) (end 150.5 121) (width 1) (layer "F.Cu") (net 7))
 (segment (start 150.5 119) (end 150.5 120) (width 1) (layer "F.Cu") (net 7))
 (segment (start 152 122.5) (end 150.5 122.5) (width 1) (layer "F.Cu") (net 7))
 (segment (start 149.5 120) (end 150.5 121) (width 1) (layer "F.Cu") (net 7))
 (segment (start 143.7 119.9) (end 149.5 119.9) (width 1) (layer "F.Cu") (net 7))
 (segment (start 149.6 119.9) (end 150.5 119) (width 1) (layer "F.Cu") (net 7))
 (segment (start 149.5 119.9) (end 149.6 119.9) (width 1) (layer "F.Cu") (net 7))
 (segment (start 153 137.6172) (end 153 123.5) (width 1) (layer "F.Cu") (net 7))
 (segment (start 149.5 119.9) (end 149.5 120) (width 1) (layer "F.Cu") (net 7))
 (segment (start 149.5 119.9) (end 150.4 119.9) (width 1) (layer "F.Cu") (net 7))
 (segment (start 150.5 116.25) (end 150.5 119) (width 1) (layer "F.Cu") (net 7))
 (segment (start 150.5 121) (end 150.5 122.5) (width 1) (layer "F.Cu") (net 7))
 (segment (start 150.4 119.9) (end 150.5 120) (width 1) (layer "F.Cu") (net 7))
 (segment (start 153 123.5) (end 152 122.5) (width 1) (layer "F.Cu") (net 7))
 (segment (start 115 120.828) (end 114.173 120.001) (width 1) (layer "F.Cu") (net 13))
 (segment (start 115.928 119.9) (end 115.827 120.001) (width 1) (layer "F.Cu") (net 13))
 (segment (start 114.173 120.001) (end 104.902 120.001) (width 1) (layer "F.Cu") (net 13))
 (segment (start 115 122.62) (end 115 120.828) (width 1) (layer "F.Cu") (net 13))
 (segment (start 114.173 120.001) (end 115.827 120.001) (width 1) (layer "F.Cu") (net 13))
 (segment (start 115.827 120.001) (end 115 120.828) (width 1) (layer "F.Cu") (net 13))
 (segment (start 125.82 120) (end 125.92 119.9) (width 1.5) (layer "F.Cu") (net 13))
 (segment (start 125.92 119.9) (end 115.928 119.9) (width 1) (layer "F.Cu") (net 13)))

